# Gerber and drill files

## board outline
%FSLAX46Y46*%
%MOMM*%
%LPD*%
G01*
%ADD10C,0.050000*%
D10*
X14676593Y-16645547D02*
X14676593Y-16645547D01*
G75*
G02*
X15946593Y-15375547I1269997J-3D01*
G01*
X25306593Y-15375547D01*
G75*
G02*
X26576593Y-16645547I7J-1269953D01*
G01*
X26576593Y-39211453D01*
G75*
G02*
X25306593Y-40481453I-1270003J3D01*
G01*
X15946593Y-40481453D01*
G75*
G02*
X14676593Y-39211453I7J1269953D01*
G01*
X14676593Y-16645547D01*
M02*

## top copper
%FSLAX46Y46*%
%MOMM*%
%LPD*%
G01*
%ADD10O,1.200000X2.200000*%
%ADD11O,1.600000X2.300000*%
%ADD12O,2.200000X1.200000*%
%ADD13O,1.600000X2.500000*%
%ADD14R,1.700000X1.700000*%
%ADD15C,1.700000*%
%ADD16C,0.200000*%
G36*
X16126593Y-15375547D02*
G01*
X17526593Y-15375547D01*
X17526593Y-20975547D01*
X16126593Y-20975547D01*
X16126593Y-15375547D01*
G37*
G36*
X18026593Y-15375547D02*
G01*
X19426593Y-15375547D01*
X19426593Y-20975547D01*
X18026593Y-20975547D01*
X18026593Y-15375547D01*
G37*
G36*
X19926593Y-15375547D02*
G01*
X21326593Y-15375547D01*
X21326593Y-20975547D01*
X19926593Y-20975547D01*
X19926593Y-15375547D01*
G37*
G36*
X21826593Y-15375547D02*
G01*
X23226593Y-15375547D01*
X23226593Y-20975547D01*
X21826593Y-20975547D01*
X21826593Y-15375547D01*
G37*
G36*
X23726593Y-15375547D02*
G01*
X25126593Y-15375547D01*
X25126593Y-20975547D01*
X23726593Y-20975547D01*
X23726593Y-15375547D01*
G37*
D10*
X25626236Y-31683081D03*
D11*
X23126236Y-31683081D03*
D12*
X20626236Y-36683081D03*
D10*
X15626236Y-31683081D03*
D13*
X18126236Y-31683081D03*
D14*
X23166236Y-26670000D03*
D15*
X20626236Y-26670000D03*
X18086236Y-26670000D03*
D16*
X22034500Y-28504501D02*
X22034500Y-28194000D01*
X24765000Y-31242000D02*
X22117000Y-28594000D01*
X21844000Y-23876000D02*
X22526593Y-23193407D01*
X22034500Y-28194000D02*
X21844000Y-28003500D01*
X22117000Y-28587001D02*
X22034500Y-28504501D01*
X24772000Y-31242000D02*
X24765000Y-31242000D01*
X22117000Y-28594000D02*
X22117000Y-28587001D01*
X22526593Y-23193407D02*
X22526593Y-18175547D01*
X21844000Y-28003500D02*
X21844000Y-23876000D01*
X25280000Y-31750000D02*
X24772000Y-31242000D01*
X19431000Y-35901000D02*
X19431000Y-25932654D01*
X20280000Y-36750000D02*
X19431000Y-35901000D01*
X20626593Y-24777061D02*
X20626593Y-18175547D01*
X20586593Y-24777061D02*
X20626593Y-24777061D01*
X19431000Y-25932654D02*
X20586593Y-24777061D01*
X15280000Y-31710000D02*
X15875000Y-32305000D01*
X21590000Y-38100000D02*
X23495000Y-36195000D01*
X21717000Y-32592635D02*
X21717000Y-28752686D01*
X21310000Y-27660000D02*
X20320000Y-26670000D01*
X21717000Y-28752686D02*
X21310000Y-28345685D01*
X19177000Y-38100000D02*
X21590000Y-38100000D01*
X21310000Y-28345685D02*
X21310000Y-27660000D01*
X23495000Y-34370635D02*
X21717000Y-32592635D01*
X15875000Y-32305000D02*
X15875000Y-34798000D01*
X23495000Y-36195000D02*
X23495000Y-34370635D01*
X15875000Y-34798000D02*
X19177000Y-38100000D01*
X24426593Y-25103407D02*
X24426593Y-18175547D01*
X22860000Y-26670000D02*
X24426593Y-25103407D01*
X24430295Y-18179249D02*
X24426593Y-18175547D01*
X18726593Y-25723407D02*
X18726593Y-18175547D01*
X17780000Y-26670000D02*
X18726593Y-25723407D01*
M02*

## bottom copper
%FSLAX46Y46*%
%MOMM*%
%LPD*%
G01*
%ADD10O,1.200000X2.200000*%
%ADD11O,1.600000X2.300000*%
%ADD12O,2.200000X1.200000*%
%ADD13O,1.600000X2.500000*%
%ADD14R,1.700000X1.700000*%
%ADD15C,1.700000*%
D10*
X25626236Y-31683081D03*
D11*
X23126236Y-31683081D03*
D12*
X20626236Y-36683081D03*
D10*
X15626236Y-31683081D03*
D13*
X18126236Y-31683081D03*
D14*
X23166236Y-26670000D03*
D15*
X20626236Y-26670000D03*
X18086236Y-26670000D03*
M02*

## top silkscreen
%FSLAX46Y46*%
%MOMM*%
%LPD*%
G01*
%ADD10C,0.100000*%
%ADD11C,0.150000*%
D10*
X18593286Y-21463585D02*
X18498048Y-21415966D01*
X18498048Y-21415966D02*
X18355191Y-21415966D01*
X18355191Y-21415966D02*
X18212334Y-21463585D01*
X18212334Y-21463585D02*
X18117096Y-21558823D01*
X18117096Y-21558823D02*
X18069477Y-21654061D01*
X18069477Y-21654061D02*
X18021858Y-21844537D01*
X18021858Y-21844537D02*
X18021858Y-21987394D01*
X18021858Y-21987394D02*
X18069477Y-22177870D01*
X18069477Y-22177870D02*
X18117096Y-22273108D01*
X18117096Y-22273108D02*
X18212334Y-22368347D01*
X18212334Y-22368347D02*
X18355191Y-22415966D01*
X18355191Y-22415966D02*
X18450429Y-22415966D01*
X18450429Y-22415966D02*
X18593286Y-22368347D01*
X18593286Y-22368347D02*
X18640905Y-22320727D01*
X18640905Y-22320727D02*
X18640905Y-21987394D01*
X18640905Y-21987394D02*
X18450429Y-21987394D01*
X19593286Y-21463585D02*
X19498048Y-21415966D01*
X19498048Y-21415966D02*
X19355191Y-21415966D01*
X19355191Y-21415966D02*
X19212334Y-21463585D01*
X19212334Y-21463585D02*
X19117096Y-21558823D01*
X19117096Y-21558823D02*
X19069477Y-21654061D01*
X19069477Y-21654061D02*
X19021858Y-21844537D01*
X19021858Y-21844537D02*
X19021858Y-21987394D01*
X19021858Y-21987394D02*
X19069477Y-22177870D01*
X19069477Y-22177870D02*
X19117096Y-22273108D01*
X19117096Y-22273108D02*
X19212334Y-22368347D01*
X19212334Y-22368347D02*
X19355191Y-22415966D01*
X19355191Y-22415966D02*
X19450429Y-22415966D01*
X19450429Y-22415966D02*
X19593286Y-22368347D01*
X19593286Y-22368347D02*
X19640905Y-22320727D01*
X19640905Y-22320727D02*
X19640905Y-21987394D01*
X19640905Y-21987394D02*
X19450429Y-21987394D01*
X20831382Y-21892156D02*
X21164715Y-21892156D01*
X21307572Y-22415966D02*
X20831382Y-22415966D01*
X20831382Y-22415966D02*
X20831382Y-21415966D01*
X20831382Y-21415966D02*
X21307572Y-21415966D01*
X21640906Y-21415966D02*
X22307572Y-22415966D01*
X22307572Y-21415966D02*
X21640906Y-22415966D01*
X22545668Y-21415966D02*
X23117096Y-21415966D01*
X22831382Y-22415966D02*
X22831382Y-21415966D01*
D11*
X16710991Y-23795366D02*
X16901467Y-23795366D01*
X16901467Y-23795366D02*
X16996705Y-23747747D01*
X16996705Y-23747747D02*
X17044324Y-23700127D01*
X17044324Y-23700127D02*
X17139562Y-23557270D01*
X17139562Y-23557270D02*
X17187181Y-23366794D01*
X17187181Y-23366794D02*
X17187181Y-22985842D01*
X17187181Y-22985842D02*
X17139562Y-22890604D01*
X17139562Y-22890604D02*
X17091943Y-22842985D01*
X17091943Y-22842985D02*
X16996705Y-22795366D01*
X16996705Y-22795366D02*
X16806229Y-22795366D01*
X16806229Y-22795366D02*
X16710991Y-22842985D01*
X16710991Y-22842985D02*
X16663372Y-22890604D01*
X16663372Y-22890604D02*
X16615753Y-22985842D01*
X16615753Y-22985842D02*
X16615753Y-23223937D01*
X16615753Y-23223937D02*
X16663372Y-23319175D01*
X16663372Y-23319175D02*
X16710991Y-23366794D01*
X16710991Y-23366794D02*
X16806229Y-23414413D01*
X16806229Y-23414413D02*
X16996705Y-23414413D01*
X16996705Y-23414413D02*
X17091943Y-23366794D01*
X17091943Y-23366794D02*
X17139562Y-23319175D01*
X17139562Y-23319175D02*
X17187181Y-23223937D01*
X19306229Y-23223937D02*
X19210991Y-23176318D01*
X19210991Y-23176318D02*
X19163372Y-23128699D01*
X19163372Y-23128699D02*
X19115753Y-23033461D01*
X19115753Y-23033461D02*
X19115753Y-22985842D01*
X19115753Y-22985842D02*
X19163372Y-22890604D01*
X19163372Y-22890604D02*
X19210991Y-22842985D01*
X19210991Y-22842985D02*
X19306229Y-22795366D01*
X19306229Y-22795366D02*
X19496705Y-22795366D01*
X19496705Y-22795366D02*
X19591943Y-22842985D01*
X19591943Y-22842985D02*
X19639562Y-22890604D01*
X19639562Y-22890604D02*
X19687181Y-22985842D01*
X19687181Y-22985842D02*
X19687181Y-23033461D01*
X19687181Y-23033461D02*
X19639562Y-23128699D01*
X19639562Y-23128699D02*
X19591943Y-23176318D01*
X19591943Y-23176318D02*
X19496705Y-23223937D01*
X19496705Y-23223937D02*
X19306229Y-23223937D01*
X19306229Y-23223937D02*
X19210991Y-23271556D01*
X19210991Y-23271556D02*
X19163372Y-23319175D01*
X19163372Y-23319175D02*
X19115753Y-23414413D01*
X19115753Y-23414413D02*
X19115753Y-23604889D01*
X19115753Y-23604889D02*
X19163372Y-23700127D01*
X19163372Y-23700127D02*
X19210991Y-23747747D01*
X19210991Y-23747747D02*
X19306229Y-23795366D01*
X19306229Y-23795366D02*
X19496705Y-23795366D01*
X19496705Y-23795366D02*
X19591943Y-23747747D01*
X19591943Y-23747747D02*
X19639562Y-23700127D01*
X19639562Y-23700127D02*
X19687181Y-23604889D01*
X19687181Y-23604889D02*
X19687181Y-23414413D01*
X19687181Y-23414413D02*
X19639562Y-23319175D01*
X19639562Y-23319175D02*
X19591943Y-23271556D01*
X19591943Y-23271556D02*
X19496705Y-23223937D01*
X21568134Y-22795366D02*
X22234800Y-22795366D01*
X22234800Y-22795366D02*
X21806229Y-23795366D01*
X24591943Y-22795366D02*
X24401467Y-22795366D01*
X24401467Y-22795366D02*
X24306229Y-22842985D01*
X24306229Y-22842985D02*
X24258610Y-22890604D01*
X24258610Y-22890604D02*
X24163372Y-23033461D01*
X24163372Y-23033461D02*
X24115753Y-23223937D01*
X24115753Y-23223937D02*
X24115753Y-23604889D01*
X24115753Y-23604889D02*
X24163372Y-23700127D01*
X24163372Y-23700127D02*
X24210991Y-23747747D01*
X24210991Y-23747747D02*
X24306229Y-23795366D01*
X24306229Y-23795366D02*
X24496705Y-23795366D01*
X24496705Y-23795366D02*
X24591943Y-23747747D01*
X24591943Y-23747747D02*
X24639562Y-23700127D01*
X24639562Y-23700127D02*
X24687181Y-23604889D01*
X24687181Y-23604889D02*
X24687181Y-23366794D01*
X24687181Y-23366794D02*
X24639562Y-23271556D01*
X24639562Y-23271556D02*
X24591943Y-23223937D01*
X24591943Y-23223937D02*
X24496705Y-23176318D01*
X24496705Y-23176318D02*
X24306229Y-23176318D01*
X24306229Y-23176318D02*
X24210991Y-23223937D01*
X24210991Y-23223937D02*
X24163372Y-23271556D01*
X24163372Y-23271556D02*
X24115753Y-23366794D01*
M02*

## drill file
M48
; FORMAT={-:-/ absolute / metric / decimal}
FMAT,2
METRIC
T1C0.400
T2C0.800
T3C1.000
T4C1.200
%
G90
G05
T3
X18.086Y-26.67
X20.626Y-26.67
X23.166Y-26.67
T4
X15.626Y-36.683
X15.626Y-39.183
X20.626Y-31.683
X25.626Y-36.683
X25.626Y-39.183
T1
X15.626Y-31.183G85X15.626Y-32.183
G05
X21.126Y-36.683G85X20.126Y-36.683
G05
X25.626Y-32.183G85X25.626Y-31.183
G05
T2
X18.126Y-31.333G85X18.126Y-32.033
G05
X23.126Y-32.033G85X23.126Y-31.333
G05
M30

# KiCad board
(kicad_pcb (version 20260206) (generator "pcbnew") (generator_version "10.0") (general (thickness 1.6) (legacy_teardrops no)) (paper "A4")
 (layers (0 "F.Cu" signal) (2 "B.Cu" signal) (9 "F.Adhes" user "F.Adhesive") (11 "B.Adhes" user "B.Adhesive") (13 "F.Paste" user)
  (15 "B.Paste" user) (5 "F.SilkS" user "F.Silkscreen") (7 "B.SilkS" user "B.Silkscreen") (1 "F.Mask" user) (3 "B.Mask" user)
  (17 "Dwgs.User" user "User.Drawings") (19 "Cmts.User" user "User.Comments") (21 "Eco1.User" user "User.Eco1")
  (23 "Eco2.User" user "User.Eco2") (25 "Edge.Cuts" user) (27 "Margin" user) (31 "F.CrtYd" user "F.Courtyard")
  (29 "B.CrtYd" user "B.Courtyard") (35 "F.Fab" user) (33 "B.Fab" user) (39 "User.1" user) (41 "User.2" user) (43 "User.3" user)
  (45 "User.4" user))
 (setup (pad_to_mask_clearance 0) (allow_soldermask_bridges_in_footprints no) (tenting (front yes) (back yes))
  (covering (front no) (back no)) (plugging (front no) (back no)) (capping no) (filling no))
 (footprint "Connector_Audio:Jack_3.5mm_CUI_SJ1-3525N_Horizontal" (layer "B.Cu") (at 20.626236 36.683081 180)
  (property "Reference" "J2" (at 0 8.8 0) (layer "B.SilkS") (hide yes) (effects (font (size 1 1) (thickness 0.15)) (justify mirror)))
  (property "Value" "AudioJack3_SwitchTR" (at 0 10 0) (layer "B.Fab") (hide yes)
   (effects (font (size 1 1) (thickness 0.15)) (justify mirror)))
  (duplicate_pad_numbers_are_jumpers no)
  (pad "" np_thru_hole circle (at -5 -2.5 180) (size 1.2 1.2) (drill 1.2) (layers "*.Cu" "*.Mask"))
  (pad "" np_thru_hole circle (at -5 0 180) (size 1.2 1.2) (drill 1.2) (layers "*.Cu" "*.Mask"))
  (pad "" np_thru_hole circle (at 0 5 180) (size 1.2 1.2) (drill 1.2) (layers "*.Cu" "*.Mask"))
  (pad "" np_thru_hole circle (at 5 -2.5 180) (size 1.2 1.2) (drill 1.2) (layers "*.Cu" "*.Mask"))
  (pad "" np_thru_hole circle (at 5 0 180) (size 1.2 1.2) (drill 1.2) (layers "*.Cu" "*.Mask"))
  (pad "R" thru_hole oval (at -5 5 180) (size 1.2 2.2) (drill oval 0.4 1.4) (layers "*.Cu" "*.Mask") (remove_unused_layers no)
   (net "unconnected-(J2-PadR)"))
  (pad "RN" thru_hole oval (at -2.5 5 180) (size 1.6 2.3) (drill oval 0.8 1.5) (layers "*.Cu" "*.Mask") (remove_unused_layers no)
   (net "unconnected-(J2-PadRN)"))
  (pad "S" thru_hole oval (at 0 0 180) (size 2.2 1.2) (drill oval 1.4 0.4) (layers "*.Cu" "*.Mask") (remove_unused_layers no)
   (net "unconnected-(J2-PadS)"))
  (pad "T" thru_hole oval (at 5 5) (size 1.2 2.2) (drill oval 0.4 1.4) (layers "*.Cu" "*.Mask") (remove_unused_layers no)
   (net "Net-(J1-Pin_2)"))
  (pad "TN" thru_hole oval (at 2.5 5) (size 1.6 2.5) (drill oval 0.8 1.5) (layers "*.Cu" "*.Mask") (remove_unused_layers no)
   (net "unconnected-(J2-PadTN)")))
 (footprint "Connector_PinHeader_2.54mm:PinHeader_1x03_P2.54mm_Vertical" (layer "B.Cu") (at 23.166236 26.67 90)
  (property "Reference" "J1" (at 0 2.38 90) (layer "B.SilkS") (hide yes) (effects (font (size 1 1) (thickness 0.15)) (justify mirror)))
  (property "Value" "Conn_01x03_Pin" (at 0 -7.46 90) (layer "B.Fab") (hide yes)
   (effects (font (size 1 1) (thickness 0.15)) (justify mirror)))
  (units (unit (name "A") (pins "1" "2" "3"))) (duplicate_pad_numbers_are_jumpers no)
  (pad "1" thru_hole rect (at 0 0 90) (size 1.7 1.7) (drill 1) (layers "*.Cu" "*.Mask") (remove_unused_layers no)
   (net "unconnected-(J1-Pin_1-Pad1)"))
  (pad "2" thru_hole circle (at 0 -2.54 90) (size 1.7 1.7) (drill 1) (layers "*.Cu" "*.Mask") (remove_unused_layers no)
   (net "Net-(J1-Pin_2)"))
  (pad "3" thru_hole circle (at 0 -5.08 90) (size 1.7 1.7) (drill 1) (layers "*.Cu" "*.Mask") (remove_unused_layers no)
   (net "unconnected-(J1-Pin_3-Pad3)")))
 (gr_rect (start 16.126593 15.375547) (end 17.526593 20.975547) (stroke (width 0) (type solid)) (fill yes) (layers "F.Cu" "F.Mask"))
 (gr_rect (start 18.026593 15.375547) (end 19.426593 20.975547) (stroke (width 0) (type solid)) (fill yes) (layers "F.Cu" "F.Mask")
  (net "unconnected-(J1-Pin_3-Pad3)"))
 (gr_rect (start 19.926593 15.375547) (end 21.326593 20.975547) (stroke (width 0) (type solid)) (fill yes) (layers "F.Cu" "F.Mask")
  (net "unconnected-(J2-PadS)"))
 (gr_rect (start 21.826593 15.375547) (end 23.226593 20.975547) (stroke (width 0) (type solid)) (fill yes) (layers "F.Cu" "F.Mask")
  (net "unconnected-(J2-PadR)"))
 (gr_rect (start 23.726593 15.375547) (end 25.126593 20.975547) (stroke (width 0) (type solid)) (fill yes) (layers "F.Cu" "F.Mask")
  (net "unconnected-(J1-Pin_1-Pad1)"))
 (gr_rect (start 14.676593 15.375547) (end 26.576593 40.481453) (radius 1.27) (stroke (width 0.05) (type solid)) (fill no)
  (layer "Edge.Cuts"))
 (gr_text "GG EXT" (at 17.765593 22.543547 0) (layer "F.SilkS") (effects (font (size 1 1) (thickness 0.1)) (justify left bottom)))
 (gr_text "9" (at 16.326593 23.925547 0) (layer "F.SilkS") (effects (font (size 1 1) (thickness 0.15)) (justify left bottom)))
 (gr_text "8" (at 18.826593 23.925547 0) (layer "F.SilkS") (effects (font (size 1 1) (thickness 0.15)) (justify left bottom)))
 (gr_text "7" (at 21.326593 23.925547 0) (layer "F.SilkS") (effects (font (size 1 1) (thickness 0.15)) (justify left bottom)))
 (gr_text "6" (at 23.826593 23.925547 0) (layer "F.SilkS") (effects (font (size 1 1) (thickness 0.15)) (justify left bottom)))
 (segment (start 22.0345 28.504501) (end 22.0345 28.194) (width 0.2) (layer "F.Cu") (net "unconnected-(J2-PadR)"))
 (segment (start 24.765 31.242) (end 22.117 28.594) (width 0.2) (layer "F.Cu") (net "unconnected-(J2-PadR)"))
 (segment (start 21.844 23.876) (end 22.526593 23.193407) (width 0.2) (layer "F.Cu") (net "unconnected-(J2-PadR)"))
 (segment (start 22.0345 28.194) (end 21.844 28.0035) (width 0.2) (layer "F.Cu") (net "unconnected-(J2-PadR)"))
 (segment (start 22.117 28.587001) (end 22.0345 28.504501) (width 0.2) (layer "F.Cu") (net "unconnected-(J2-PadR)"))
 (segment (start 24.772 31.242) (end 24.765 31.242) (width 0.2) (layer "F.Cu") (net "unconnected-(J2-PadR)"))
 (segment (start 22.117 28.594) (end 22.117 28.587001) (width 0.2) (layer "F.Cu") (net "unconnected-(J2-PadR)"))
 (segment (start 22.526593 23.193407) (end 22.526593 18.175547) (width 0.2) (layer "F.Cu") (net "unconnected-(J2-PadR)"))
 (segment (start 21.844 28.0035) (end 21.844 23.876) (width 0.2) (layer "F.Cu") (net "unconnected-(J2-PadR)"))
 (segment (start 25.28 31.75) (end 24.772 31.242) (width 0.2) (layer "F.Cu") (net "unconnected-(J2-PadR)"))
 (segment (start 19.431 35.901) (end 19.431 25.932654) (width 0.2) (layer "F.Cu") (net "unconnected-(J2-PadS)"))
 (segment (start 20.28 36.75) (end 19.431 35.901) (width 0.2) (layer "F.Cu") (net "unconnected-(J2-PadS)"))
 (segment (start 20.626593 24.777061) (end 20.626593 18.175547) (width 0.2) (layer "F.Cu") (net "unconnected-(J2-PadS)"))
 (segment (start 20.586593 24.777061) (end 20.626593 24.777061) (width 0.2) (layer "F.Cu") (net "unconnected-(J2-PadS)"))
 (segment (start 19.431 25.932654) (end 20.586593 24.777061) (width 0.2) (layer "F.Cu") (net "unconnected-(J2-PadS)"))
 (segment (start 15.28 31.71) (end 15.875 32.305) (width 0.2) (layer "F.Cu") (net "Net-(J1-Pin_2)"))
 (segment (start 21.59 38.1) (end 23.495 36.195) (width 0.2) (layer "F.Cu") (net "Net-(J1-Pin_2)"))
 (segment (start 21.717 32.592635) (end 21.717 28.752686) (width 0.2) (layer "F.Cu") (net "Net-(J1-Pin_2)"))
 (segment (start 21.31 27.66) (end 20.32 26.67) (width 0.2) (layer "F.Cu") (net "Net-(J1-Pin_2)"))
 (segment (start 21.717 28.752686) (end 21.31 28.345685) (width 0.2) (layer "F.Cu") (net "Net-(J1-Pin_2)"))
 (segment (start 19.177 38.1) (end 21.59 38.1) (width 0.2) (layer "F.Cu") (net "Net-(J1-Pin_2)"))
 (segment (start 21.31 28.345685) (end 21.31 27.66) (width 0.2) (layer "F.Cu") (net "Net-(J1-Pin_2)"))
 (segment (start 23.495 34.370635) (end 21.717 32.592635) (width 0.2) (layer "F.Cu") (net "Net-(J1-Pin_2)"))
 (segment (start 15.875 32.305) (end 15.875 34.798) (width 0.2) (layer "F.Cu") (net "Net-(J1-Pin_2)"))
 (segment (start 23.495 36.195) (end 23.495 34.370635) (width 0.2) (layer "F.Cu") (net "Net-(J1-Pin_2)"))
 (segment (start 15.875 34.798) (end 19.177 38.1) (width 0.2) (layer "F.Cu") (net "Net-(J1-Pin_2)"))
 (segment (start 24.426593 25.103407) (end 24.426593 18.175547) (width 0.2) (layer "F.Cu") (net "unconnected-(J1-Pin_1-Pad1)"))
 (segment (start 22.86 26.67) (end 24.426593 25.103407) (width 0.2) (layer "F.Cu") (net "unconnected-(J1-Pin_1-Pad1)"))
 (segment (start 24.430295 18.179249) (end 24.426593 18.175547) (width 0.2) (layer "F.Cu") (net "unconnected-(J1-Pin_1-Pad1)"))
 (segment (start 18.726593 25.723407) (end 18.726593 18.175547) (width 0.2) (layer "F.Cu") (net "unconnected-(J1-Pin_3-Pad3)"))
 (segment (start 17.78 26.67) (end 18.726593 25.723407) (width 0.2) (layer "F.Cu") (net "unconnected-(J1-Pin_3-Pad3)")))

